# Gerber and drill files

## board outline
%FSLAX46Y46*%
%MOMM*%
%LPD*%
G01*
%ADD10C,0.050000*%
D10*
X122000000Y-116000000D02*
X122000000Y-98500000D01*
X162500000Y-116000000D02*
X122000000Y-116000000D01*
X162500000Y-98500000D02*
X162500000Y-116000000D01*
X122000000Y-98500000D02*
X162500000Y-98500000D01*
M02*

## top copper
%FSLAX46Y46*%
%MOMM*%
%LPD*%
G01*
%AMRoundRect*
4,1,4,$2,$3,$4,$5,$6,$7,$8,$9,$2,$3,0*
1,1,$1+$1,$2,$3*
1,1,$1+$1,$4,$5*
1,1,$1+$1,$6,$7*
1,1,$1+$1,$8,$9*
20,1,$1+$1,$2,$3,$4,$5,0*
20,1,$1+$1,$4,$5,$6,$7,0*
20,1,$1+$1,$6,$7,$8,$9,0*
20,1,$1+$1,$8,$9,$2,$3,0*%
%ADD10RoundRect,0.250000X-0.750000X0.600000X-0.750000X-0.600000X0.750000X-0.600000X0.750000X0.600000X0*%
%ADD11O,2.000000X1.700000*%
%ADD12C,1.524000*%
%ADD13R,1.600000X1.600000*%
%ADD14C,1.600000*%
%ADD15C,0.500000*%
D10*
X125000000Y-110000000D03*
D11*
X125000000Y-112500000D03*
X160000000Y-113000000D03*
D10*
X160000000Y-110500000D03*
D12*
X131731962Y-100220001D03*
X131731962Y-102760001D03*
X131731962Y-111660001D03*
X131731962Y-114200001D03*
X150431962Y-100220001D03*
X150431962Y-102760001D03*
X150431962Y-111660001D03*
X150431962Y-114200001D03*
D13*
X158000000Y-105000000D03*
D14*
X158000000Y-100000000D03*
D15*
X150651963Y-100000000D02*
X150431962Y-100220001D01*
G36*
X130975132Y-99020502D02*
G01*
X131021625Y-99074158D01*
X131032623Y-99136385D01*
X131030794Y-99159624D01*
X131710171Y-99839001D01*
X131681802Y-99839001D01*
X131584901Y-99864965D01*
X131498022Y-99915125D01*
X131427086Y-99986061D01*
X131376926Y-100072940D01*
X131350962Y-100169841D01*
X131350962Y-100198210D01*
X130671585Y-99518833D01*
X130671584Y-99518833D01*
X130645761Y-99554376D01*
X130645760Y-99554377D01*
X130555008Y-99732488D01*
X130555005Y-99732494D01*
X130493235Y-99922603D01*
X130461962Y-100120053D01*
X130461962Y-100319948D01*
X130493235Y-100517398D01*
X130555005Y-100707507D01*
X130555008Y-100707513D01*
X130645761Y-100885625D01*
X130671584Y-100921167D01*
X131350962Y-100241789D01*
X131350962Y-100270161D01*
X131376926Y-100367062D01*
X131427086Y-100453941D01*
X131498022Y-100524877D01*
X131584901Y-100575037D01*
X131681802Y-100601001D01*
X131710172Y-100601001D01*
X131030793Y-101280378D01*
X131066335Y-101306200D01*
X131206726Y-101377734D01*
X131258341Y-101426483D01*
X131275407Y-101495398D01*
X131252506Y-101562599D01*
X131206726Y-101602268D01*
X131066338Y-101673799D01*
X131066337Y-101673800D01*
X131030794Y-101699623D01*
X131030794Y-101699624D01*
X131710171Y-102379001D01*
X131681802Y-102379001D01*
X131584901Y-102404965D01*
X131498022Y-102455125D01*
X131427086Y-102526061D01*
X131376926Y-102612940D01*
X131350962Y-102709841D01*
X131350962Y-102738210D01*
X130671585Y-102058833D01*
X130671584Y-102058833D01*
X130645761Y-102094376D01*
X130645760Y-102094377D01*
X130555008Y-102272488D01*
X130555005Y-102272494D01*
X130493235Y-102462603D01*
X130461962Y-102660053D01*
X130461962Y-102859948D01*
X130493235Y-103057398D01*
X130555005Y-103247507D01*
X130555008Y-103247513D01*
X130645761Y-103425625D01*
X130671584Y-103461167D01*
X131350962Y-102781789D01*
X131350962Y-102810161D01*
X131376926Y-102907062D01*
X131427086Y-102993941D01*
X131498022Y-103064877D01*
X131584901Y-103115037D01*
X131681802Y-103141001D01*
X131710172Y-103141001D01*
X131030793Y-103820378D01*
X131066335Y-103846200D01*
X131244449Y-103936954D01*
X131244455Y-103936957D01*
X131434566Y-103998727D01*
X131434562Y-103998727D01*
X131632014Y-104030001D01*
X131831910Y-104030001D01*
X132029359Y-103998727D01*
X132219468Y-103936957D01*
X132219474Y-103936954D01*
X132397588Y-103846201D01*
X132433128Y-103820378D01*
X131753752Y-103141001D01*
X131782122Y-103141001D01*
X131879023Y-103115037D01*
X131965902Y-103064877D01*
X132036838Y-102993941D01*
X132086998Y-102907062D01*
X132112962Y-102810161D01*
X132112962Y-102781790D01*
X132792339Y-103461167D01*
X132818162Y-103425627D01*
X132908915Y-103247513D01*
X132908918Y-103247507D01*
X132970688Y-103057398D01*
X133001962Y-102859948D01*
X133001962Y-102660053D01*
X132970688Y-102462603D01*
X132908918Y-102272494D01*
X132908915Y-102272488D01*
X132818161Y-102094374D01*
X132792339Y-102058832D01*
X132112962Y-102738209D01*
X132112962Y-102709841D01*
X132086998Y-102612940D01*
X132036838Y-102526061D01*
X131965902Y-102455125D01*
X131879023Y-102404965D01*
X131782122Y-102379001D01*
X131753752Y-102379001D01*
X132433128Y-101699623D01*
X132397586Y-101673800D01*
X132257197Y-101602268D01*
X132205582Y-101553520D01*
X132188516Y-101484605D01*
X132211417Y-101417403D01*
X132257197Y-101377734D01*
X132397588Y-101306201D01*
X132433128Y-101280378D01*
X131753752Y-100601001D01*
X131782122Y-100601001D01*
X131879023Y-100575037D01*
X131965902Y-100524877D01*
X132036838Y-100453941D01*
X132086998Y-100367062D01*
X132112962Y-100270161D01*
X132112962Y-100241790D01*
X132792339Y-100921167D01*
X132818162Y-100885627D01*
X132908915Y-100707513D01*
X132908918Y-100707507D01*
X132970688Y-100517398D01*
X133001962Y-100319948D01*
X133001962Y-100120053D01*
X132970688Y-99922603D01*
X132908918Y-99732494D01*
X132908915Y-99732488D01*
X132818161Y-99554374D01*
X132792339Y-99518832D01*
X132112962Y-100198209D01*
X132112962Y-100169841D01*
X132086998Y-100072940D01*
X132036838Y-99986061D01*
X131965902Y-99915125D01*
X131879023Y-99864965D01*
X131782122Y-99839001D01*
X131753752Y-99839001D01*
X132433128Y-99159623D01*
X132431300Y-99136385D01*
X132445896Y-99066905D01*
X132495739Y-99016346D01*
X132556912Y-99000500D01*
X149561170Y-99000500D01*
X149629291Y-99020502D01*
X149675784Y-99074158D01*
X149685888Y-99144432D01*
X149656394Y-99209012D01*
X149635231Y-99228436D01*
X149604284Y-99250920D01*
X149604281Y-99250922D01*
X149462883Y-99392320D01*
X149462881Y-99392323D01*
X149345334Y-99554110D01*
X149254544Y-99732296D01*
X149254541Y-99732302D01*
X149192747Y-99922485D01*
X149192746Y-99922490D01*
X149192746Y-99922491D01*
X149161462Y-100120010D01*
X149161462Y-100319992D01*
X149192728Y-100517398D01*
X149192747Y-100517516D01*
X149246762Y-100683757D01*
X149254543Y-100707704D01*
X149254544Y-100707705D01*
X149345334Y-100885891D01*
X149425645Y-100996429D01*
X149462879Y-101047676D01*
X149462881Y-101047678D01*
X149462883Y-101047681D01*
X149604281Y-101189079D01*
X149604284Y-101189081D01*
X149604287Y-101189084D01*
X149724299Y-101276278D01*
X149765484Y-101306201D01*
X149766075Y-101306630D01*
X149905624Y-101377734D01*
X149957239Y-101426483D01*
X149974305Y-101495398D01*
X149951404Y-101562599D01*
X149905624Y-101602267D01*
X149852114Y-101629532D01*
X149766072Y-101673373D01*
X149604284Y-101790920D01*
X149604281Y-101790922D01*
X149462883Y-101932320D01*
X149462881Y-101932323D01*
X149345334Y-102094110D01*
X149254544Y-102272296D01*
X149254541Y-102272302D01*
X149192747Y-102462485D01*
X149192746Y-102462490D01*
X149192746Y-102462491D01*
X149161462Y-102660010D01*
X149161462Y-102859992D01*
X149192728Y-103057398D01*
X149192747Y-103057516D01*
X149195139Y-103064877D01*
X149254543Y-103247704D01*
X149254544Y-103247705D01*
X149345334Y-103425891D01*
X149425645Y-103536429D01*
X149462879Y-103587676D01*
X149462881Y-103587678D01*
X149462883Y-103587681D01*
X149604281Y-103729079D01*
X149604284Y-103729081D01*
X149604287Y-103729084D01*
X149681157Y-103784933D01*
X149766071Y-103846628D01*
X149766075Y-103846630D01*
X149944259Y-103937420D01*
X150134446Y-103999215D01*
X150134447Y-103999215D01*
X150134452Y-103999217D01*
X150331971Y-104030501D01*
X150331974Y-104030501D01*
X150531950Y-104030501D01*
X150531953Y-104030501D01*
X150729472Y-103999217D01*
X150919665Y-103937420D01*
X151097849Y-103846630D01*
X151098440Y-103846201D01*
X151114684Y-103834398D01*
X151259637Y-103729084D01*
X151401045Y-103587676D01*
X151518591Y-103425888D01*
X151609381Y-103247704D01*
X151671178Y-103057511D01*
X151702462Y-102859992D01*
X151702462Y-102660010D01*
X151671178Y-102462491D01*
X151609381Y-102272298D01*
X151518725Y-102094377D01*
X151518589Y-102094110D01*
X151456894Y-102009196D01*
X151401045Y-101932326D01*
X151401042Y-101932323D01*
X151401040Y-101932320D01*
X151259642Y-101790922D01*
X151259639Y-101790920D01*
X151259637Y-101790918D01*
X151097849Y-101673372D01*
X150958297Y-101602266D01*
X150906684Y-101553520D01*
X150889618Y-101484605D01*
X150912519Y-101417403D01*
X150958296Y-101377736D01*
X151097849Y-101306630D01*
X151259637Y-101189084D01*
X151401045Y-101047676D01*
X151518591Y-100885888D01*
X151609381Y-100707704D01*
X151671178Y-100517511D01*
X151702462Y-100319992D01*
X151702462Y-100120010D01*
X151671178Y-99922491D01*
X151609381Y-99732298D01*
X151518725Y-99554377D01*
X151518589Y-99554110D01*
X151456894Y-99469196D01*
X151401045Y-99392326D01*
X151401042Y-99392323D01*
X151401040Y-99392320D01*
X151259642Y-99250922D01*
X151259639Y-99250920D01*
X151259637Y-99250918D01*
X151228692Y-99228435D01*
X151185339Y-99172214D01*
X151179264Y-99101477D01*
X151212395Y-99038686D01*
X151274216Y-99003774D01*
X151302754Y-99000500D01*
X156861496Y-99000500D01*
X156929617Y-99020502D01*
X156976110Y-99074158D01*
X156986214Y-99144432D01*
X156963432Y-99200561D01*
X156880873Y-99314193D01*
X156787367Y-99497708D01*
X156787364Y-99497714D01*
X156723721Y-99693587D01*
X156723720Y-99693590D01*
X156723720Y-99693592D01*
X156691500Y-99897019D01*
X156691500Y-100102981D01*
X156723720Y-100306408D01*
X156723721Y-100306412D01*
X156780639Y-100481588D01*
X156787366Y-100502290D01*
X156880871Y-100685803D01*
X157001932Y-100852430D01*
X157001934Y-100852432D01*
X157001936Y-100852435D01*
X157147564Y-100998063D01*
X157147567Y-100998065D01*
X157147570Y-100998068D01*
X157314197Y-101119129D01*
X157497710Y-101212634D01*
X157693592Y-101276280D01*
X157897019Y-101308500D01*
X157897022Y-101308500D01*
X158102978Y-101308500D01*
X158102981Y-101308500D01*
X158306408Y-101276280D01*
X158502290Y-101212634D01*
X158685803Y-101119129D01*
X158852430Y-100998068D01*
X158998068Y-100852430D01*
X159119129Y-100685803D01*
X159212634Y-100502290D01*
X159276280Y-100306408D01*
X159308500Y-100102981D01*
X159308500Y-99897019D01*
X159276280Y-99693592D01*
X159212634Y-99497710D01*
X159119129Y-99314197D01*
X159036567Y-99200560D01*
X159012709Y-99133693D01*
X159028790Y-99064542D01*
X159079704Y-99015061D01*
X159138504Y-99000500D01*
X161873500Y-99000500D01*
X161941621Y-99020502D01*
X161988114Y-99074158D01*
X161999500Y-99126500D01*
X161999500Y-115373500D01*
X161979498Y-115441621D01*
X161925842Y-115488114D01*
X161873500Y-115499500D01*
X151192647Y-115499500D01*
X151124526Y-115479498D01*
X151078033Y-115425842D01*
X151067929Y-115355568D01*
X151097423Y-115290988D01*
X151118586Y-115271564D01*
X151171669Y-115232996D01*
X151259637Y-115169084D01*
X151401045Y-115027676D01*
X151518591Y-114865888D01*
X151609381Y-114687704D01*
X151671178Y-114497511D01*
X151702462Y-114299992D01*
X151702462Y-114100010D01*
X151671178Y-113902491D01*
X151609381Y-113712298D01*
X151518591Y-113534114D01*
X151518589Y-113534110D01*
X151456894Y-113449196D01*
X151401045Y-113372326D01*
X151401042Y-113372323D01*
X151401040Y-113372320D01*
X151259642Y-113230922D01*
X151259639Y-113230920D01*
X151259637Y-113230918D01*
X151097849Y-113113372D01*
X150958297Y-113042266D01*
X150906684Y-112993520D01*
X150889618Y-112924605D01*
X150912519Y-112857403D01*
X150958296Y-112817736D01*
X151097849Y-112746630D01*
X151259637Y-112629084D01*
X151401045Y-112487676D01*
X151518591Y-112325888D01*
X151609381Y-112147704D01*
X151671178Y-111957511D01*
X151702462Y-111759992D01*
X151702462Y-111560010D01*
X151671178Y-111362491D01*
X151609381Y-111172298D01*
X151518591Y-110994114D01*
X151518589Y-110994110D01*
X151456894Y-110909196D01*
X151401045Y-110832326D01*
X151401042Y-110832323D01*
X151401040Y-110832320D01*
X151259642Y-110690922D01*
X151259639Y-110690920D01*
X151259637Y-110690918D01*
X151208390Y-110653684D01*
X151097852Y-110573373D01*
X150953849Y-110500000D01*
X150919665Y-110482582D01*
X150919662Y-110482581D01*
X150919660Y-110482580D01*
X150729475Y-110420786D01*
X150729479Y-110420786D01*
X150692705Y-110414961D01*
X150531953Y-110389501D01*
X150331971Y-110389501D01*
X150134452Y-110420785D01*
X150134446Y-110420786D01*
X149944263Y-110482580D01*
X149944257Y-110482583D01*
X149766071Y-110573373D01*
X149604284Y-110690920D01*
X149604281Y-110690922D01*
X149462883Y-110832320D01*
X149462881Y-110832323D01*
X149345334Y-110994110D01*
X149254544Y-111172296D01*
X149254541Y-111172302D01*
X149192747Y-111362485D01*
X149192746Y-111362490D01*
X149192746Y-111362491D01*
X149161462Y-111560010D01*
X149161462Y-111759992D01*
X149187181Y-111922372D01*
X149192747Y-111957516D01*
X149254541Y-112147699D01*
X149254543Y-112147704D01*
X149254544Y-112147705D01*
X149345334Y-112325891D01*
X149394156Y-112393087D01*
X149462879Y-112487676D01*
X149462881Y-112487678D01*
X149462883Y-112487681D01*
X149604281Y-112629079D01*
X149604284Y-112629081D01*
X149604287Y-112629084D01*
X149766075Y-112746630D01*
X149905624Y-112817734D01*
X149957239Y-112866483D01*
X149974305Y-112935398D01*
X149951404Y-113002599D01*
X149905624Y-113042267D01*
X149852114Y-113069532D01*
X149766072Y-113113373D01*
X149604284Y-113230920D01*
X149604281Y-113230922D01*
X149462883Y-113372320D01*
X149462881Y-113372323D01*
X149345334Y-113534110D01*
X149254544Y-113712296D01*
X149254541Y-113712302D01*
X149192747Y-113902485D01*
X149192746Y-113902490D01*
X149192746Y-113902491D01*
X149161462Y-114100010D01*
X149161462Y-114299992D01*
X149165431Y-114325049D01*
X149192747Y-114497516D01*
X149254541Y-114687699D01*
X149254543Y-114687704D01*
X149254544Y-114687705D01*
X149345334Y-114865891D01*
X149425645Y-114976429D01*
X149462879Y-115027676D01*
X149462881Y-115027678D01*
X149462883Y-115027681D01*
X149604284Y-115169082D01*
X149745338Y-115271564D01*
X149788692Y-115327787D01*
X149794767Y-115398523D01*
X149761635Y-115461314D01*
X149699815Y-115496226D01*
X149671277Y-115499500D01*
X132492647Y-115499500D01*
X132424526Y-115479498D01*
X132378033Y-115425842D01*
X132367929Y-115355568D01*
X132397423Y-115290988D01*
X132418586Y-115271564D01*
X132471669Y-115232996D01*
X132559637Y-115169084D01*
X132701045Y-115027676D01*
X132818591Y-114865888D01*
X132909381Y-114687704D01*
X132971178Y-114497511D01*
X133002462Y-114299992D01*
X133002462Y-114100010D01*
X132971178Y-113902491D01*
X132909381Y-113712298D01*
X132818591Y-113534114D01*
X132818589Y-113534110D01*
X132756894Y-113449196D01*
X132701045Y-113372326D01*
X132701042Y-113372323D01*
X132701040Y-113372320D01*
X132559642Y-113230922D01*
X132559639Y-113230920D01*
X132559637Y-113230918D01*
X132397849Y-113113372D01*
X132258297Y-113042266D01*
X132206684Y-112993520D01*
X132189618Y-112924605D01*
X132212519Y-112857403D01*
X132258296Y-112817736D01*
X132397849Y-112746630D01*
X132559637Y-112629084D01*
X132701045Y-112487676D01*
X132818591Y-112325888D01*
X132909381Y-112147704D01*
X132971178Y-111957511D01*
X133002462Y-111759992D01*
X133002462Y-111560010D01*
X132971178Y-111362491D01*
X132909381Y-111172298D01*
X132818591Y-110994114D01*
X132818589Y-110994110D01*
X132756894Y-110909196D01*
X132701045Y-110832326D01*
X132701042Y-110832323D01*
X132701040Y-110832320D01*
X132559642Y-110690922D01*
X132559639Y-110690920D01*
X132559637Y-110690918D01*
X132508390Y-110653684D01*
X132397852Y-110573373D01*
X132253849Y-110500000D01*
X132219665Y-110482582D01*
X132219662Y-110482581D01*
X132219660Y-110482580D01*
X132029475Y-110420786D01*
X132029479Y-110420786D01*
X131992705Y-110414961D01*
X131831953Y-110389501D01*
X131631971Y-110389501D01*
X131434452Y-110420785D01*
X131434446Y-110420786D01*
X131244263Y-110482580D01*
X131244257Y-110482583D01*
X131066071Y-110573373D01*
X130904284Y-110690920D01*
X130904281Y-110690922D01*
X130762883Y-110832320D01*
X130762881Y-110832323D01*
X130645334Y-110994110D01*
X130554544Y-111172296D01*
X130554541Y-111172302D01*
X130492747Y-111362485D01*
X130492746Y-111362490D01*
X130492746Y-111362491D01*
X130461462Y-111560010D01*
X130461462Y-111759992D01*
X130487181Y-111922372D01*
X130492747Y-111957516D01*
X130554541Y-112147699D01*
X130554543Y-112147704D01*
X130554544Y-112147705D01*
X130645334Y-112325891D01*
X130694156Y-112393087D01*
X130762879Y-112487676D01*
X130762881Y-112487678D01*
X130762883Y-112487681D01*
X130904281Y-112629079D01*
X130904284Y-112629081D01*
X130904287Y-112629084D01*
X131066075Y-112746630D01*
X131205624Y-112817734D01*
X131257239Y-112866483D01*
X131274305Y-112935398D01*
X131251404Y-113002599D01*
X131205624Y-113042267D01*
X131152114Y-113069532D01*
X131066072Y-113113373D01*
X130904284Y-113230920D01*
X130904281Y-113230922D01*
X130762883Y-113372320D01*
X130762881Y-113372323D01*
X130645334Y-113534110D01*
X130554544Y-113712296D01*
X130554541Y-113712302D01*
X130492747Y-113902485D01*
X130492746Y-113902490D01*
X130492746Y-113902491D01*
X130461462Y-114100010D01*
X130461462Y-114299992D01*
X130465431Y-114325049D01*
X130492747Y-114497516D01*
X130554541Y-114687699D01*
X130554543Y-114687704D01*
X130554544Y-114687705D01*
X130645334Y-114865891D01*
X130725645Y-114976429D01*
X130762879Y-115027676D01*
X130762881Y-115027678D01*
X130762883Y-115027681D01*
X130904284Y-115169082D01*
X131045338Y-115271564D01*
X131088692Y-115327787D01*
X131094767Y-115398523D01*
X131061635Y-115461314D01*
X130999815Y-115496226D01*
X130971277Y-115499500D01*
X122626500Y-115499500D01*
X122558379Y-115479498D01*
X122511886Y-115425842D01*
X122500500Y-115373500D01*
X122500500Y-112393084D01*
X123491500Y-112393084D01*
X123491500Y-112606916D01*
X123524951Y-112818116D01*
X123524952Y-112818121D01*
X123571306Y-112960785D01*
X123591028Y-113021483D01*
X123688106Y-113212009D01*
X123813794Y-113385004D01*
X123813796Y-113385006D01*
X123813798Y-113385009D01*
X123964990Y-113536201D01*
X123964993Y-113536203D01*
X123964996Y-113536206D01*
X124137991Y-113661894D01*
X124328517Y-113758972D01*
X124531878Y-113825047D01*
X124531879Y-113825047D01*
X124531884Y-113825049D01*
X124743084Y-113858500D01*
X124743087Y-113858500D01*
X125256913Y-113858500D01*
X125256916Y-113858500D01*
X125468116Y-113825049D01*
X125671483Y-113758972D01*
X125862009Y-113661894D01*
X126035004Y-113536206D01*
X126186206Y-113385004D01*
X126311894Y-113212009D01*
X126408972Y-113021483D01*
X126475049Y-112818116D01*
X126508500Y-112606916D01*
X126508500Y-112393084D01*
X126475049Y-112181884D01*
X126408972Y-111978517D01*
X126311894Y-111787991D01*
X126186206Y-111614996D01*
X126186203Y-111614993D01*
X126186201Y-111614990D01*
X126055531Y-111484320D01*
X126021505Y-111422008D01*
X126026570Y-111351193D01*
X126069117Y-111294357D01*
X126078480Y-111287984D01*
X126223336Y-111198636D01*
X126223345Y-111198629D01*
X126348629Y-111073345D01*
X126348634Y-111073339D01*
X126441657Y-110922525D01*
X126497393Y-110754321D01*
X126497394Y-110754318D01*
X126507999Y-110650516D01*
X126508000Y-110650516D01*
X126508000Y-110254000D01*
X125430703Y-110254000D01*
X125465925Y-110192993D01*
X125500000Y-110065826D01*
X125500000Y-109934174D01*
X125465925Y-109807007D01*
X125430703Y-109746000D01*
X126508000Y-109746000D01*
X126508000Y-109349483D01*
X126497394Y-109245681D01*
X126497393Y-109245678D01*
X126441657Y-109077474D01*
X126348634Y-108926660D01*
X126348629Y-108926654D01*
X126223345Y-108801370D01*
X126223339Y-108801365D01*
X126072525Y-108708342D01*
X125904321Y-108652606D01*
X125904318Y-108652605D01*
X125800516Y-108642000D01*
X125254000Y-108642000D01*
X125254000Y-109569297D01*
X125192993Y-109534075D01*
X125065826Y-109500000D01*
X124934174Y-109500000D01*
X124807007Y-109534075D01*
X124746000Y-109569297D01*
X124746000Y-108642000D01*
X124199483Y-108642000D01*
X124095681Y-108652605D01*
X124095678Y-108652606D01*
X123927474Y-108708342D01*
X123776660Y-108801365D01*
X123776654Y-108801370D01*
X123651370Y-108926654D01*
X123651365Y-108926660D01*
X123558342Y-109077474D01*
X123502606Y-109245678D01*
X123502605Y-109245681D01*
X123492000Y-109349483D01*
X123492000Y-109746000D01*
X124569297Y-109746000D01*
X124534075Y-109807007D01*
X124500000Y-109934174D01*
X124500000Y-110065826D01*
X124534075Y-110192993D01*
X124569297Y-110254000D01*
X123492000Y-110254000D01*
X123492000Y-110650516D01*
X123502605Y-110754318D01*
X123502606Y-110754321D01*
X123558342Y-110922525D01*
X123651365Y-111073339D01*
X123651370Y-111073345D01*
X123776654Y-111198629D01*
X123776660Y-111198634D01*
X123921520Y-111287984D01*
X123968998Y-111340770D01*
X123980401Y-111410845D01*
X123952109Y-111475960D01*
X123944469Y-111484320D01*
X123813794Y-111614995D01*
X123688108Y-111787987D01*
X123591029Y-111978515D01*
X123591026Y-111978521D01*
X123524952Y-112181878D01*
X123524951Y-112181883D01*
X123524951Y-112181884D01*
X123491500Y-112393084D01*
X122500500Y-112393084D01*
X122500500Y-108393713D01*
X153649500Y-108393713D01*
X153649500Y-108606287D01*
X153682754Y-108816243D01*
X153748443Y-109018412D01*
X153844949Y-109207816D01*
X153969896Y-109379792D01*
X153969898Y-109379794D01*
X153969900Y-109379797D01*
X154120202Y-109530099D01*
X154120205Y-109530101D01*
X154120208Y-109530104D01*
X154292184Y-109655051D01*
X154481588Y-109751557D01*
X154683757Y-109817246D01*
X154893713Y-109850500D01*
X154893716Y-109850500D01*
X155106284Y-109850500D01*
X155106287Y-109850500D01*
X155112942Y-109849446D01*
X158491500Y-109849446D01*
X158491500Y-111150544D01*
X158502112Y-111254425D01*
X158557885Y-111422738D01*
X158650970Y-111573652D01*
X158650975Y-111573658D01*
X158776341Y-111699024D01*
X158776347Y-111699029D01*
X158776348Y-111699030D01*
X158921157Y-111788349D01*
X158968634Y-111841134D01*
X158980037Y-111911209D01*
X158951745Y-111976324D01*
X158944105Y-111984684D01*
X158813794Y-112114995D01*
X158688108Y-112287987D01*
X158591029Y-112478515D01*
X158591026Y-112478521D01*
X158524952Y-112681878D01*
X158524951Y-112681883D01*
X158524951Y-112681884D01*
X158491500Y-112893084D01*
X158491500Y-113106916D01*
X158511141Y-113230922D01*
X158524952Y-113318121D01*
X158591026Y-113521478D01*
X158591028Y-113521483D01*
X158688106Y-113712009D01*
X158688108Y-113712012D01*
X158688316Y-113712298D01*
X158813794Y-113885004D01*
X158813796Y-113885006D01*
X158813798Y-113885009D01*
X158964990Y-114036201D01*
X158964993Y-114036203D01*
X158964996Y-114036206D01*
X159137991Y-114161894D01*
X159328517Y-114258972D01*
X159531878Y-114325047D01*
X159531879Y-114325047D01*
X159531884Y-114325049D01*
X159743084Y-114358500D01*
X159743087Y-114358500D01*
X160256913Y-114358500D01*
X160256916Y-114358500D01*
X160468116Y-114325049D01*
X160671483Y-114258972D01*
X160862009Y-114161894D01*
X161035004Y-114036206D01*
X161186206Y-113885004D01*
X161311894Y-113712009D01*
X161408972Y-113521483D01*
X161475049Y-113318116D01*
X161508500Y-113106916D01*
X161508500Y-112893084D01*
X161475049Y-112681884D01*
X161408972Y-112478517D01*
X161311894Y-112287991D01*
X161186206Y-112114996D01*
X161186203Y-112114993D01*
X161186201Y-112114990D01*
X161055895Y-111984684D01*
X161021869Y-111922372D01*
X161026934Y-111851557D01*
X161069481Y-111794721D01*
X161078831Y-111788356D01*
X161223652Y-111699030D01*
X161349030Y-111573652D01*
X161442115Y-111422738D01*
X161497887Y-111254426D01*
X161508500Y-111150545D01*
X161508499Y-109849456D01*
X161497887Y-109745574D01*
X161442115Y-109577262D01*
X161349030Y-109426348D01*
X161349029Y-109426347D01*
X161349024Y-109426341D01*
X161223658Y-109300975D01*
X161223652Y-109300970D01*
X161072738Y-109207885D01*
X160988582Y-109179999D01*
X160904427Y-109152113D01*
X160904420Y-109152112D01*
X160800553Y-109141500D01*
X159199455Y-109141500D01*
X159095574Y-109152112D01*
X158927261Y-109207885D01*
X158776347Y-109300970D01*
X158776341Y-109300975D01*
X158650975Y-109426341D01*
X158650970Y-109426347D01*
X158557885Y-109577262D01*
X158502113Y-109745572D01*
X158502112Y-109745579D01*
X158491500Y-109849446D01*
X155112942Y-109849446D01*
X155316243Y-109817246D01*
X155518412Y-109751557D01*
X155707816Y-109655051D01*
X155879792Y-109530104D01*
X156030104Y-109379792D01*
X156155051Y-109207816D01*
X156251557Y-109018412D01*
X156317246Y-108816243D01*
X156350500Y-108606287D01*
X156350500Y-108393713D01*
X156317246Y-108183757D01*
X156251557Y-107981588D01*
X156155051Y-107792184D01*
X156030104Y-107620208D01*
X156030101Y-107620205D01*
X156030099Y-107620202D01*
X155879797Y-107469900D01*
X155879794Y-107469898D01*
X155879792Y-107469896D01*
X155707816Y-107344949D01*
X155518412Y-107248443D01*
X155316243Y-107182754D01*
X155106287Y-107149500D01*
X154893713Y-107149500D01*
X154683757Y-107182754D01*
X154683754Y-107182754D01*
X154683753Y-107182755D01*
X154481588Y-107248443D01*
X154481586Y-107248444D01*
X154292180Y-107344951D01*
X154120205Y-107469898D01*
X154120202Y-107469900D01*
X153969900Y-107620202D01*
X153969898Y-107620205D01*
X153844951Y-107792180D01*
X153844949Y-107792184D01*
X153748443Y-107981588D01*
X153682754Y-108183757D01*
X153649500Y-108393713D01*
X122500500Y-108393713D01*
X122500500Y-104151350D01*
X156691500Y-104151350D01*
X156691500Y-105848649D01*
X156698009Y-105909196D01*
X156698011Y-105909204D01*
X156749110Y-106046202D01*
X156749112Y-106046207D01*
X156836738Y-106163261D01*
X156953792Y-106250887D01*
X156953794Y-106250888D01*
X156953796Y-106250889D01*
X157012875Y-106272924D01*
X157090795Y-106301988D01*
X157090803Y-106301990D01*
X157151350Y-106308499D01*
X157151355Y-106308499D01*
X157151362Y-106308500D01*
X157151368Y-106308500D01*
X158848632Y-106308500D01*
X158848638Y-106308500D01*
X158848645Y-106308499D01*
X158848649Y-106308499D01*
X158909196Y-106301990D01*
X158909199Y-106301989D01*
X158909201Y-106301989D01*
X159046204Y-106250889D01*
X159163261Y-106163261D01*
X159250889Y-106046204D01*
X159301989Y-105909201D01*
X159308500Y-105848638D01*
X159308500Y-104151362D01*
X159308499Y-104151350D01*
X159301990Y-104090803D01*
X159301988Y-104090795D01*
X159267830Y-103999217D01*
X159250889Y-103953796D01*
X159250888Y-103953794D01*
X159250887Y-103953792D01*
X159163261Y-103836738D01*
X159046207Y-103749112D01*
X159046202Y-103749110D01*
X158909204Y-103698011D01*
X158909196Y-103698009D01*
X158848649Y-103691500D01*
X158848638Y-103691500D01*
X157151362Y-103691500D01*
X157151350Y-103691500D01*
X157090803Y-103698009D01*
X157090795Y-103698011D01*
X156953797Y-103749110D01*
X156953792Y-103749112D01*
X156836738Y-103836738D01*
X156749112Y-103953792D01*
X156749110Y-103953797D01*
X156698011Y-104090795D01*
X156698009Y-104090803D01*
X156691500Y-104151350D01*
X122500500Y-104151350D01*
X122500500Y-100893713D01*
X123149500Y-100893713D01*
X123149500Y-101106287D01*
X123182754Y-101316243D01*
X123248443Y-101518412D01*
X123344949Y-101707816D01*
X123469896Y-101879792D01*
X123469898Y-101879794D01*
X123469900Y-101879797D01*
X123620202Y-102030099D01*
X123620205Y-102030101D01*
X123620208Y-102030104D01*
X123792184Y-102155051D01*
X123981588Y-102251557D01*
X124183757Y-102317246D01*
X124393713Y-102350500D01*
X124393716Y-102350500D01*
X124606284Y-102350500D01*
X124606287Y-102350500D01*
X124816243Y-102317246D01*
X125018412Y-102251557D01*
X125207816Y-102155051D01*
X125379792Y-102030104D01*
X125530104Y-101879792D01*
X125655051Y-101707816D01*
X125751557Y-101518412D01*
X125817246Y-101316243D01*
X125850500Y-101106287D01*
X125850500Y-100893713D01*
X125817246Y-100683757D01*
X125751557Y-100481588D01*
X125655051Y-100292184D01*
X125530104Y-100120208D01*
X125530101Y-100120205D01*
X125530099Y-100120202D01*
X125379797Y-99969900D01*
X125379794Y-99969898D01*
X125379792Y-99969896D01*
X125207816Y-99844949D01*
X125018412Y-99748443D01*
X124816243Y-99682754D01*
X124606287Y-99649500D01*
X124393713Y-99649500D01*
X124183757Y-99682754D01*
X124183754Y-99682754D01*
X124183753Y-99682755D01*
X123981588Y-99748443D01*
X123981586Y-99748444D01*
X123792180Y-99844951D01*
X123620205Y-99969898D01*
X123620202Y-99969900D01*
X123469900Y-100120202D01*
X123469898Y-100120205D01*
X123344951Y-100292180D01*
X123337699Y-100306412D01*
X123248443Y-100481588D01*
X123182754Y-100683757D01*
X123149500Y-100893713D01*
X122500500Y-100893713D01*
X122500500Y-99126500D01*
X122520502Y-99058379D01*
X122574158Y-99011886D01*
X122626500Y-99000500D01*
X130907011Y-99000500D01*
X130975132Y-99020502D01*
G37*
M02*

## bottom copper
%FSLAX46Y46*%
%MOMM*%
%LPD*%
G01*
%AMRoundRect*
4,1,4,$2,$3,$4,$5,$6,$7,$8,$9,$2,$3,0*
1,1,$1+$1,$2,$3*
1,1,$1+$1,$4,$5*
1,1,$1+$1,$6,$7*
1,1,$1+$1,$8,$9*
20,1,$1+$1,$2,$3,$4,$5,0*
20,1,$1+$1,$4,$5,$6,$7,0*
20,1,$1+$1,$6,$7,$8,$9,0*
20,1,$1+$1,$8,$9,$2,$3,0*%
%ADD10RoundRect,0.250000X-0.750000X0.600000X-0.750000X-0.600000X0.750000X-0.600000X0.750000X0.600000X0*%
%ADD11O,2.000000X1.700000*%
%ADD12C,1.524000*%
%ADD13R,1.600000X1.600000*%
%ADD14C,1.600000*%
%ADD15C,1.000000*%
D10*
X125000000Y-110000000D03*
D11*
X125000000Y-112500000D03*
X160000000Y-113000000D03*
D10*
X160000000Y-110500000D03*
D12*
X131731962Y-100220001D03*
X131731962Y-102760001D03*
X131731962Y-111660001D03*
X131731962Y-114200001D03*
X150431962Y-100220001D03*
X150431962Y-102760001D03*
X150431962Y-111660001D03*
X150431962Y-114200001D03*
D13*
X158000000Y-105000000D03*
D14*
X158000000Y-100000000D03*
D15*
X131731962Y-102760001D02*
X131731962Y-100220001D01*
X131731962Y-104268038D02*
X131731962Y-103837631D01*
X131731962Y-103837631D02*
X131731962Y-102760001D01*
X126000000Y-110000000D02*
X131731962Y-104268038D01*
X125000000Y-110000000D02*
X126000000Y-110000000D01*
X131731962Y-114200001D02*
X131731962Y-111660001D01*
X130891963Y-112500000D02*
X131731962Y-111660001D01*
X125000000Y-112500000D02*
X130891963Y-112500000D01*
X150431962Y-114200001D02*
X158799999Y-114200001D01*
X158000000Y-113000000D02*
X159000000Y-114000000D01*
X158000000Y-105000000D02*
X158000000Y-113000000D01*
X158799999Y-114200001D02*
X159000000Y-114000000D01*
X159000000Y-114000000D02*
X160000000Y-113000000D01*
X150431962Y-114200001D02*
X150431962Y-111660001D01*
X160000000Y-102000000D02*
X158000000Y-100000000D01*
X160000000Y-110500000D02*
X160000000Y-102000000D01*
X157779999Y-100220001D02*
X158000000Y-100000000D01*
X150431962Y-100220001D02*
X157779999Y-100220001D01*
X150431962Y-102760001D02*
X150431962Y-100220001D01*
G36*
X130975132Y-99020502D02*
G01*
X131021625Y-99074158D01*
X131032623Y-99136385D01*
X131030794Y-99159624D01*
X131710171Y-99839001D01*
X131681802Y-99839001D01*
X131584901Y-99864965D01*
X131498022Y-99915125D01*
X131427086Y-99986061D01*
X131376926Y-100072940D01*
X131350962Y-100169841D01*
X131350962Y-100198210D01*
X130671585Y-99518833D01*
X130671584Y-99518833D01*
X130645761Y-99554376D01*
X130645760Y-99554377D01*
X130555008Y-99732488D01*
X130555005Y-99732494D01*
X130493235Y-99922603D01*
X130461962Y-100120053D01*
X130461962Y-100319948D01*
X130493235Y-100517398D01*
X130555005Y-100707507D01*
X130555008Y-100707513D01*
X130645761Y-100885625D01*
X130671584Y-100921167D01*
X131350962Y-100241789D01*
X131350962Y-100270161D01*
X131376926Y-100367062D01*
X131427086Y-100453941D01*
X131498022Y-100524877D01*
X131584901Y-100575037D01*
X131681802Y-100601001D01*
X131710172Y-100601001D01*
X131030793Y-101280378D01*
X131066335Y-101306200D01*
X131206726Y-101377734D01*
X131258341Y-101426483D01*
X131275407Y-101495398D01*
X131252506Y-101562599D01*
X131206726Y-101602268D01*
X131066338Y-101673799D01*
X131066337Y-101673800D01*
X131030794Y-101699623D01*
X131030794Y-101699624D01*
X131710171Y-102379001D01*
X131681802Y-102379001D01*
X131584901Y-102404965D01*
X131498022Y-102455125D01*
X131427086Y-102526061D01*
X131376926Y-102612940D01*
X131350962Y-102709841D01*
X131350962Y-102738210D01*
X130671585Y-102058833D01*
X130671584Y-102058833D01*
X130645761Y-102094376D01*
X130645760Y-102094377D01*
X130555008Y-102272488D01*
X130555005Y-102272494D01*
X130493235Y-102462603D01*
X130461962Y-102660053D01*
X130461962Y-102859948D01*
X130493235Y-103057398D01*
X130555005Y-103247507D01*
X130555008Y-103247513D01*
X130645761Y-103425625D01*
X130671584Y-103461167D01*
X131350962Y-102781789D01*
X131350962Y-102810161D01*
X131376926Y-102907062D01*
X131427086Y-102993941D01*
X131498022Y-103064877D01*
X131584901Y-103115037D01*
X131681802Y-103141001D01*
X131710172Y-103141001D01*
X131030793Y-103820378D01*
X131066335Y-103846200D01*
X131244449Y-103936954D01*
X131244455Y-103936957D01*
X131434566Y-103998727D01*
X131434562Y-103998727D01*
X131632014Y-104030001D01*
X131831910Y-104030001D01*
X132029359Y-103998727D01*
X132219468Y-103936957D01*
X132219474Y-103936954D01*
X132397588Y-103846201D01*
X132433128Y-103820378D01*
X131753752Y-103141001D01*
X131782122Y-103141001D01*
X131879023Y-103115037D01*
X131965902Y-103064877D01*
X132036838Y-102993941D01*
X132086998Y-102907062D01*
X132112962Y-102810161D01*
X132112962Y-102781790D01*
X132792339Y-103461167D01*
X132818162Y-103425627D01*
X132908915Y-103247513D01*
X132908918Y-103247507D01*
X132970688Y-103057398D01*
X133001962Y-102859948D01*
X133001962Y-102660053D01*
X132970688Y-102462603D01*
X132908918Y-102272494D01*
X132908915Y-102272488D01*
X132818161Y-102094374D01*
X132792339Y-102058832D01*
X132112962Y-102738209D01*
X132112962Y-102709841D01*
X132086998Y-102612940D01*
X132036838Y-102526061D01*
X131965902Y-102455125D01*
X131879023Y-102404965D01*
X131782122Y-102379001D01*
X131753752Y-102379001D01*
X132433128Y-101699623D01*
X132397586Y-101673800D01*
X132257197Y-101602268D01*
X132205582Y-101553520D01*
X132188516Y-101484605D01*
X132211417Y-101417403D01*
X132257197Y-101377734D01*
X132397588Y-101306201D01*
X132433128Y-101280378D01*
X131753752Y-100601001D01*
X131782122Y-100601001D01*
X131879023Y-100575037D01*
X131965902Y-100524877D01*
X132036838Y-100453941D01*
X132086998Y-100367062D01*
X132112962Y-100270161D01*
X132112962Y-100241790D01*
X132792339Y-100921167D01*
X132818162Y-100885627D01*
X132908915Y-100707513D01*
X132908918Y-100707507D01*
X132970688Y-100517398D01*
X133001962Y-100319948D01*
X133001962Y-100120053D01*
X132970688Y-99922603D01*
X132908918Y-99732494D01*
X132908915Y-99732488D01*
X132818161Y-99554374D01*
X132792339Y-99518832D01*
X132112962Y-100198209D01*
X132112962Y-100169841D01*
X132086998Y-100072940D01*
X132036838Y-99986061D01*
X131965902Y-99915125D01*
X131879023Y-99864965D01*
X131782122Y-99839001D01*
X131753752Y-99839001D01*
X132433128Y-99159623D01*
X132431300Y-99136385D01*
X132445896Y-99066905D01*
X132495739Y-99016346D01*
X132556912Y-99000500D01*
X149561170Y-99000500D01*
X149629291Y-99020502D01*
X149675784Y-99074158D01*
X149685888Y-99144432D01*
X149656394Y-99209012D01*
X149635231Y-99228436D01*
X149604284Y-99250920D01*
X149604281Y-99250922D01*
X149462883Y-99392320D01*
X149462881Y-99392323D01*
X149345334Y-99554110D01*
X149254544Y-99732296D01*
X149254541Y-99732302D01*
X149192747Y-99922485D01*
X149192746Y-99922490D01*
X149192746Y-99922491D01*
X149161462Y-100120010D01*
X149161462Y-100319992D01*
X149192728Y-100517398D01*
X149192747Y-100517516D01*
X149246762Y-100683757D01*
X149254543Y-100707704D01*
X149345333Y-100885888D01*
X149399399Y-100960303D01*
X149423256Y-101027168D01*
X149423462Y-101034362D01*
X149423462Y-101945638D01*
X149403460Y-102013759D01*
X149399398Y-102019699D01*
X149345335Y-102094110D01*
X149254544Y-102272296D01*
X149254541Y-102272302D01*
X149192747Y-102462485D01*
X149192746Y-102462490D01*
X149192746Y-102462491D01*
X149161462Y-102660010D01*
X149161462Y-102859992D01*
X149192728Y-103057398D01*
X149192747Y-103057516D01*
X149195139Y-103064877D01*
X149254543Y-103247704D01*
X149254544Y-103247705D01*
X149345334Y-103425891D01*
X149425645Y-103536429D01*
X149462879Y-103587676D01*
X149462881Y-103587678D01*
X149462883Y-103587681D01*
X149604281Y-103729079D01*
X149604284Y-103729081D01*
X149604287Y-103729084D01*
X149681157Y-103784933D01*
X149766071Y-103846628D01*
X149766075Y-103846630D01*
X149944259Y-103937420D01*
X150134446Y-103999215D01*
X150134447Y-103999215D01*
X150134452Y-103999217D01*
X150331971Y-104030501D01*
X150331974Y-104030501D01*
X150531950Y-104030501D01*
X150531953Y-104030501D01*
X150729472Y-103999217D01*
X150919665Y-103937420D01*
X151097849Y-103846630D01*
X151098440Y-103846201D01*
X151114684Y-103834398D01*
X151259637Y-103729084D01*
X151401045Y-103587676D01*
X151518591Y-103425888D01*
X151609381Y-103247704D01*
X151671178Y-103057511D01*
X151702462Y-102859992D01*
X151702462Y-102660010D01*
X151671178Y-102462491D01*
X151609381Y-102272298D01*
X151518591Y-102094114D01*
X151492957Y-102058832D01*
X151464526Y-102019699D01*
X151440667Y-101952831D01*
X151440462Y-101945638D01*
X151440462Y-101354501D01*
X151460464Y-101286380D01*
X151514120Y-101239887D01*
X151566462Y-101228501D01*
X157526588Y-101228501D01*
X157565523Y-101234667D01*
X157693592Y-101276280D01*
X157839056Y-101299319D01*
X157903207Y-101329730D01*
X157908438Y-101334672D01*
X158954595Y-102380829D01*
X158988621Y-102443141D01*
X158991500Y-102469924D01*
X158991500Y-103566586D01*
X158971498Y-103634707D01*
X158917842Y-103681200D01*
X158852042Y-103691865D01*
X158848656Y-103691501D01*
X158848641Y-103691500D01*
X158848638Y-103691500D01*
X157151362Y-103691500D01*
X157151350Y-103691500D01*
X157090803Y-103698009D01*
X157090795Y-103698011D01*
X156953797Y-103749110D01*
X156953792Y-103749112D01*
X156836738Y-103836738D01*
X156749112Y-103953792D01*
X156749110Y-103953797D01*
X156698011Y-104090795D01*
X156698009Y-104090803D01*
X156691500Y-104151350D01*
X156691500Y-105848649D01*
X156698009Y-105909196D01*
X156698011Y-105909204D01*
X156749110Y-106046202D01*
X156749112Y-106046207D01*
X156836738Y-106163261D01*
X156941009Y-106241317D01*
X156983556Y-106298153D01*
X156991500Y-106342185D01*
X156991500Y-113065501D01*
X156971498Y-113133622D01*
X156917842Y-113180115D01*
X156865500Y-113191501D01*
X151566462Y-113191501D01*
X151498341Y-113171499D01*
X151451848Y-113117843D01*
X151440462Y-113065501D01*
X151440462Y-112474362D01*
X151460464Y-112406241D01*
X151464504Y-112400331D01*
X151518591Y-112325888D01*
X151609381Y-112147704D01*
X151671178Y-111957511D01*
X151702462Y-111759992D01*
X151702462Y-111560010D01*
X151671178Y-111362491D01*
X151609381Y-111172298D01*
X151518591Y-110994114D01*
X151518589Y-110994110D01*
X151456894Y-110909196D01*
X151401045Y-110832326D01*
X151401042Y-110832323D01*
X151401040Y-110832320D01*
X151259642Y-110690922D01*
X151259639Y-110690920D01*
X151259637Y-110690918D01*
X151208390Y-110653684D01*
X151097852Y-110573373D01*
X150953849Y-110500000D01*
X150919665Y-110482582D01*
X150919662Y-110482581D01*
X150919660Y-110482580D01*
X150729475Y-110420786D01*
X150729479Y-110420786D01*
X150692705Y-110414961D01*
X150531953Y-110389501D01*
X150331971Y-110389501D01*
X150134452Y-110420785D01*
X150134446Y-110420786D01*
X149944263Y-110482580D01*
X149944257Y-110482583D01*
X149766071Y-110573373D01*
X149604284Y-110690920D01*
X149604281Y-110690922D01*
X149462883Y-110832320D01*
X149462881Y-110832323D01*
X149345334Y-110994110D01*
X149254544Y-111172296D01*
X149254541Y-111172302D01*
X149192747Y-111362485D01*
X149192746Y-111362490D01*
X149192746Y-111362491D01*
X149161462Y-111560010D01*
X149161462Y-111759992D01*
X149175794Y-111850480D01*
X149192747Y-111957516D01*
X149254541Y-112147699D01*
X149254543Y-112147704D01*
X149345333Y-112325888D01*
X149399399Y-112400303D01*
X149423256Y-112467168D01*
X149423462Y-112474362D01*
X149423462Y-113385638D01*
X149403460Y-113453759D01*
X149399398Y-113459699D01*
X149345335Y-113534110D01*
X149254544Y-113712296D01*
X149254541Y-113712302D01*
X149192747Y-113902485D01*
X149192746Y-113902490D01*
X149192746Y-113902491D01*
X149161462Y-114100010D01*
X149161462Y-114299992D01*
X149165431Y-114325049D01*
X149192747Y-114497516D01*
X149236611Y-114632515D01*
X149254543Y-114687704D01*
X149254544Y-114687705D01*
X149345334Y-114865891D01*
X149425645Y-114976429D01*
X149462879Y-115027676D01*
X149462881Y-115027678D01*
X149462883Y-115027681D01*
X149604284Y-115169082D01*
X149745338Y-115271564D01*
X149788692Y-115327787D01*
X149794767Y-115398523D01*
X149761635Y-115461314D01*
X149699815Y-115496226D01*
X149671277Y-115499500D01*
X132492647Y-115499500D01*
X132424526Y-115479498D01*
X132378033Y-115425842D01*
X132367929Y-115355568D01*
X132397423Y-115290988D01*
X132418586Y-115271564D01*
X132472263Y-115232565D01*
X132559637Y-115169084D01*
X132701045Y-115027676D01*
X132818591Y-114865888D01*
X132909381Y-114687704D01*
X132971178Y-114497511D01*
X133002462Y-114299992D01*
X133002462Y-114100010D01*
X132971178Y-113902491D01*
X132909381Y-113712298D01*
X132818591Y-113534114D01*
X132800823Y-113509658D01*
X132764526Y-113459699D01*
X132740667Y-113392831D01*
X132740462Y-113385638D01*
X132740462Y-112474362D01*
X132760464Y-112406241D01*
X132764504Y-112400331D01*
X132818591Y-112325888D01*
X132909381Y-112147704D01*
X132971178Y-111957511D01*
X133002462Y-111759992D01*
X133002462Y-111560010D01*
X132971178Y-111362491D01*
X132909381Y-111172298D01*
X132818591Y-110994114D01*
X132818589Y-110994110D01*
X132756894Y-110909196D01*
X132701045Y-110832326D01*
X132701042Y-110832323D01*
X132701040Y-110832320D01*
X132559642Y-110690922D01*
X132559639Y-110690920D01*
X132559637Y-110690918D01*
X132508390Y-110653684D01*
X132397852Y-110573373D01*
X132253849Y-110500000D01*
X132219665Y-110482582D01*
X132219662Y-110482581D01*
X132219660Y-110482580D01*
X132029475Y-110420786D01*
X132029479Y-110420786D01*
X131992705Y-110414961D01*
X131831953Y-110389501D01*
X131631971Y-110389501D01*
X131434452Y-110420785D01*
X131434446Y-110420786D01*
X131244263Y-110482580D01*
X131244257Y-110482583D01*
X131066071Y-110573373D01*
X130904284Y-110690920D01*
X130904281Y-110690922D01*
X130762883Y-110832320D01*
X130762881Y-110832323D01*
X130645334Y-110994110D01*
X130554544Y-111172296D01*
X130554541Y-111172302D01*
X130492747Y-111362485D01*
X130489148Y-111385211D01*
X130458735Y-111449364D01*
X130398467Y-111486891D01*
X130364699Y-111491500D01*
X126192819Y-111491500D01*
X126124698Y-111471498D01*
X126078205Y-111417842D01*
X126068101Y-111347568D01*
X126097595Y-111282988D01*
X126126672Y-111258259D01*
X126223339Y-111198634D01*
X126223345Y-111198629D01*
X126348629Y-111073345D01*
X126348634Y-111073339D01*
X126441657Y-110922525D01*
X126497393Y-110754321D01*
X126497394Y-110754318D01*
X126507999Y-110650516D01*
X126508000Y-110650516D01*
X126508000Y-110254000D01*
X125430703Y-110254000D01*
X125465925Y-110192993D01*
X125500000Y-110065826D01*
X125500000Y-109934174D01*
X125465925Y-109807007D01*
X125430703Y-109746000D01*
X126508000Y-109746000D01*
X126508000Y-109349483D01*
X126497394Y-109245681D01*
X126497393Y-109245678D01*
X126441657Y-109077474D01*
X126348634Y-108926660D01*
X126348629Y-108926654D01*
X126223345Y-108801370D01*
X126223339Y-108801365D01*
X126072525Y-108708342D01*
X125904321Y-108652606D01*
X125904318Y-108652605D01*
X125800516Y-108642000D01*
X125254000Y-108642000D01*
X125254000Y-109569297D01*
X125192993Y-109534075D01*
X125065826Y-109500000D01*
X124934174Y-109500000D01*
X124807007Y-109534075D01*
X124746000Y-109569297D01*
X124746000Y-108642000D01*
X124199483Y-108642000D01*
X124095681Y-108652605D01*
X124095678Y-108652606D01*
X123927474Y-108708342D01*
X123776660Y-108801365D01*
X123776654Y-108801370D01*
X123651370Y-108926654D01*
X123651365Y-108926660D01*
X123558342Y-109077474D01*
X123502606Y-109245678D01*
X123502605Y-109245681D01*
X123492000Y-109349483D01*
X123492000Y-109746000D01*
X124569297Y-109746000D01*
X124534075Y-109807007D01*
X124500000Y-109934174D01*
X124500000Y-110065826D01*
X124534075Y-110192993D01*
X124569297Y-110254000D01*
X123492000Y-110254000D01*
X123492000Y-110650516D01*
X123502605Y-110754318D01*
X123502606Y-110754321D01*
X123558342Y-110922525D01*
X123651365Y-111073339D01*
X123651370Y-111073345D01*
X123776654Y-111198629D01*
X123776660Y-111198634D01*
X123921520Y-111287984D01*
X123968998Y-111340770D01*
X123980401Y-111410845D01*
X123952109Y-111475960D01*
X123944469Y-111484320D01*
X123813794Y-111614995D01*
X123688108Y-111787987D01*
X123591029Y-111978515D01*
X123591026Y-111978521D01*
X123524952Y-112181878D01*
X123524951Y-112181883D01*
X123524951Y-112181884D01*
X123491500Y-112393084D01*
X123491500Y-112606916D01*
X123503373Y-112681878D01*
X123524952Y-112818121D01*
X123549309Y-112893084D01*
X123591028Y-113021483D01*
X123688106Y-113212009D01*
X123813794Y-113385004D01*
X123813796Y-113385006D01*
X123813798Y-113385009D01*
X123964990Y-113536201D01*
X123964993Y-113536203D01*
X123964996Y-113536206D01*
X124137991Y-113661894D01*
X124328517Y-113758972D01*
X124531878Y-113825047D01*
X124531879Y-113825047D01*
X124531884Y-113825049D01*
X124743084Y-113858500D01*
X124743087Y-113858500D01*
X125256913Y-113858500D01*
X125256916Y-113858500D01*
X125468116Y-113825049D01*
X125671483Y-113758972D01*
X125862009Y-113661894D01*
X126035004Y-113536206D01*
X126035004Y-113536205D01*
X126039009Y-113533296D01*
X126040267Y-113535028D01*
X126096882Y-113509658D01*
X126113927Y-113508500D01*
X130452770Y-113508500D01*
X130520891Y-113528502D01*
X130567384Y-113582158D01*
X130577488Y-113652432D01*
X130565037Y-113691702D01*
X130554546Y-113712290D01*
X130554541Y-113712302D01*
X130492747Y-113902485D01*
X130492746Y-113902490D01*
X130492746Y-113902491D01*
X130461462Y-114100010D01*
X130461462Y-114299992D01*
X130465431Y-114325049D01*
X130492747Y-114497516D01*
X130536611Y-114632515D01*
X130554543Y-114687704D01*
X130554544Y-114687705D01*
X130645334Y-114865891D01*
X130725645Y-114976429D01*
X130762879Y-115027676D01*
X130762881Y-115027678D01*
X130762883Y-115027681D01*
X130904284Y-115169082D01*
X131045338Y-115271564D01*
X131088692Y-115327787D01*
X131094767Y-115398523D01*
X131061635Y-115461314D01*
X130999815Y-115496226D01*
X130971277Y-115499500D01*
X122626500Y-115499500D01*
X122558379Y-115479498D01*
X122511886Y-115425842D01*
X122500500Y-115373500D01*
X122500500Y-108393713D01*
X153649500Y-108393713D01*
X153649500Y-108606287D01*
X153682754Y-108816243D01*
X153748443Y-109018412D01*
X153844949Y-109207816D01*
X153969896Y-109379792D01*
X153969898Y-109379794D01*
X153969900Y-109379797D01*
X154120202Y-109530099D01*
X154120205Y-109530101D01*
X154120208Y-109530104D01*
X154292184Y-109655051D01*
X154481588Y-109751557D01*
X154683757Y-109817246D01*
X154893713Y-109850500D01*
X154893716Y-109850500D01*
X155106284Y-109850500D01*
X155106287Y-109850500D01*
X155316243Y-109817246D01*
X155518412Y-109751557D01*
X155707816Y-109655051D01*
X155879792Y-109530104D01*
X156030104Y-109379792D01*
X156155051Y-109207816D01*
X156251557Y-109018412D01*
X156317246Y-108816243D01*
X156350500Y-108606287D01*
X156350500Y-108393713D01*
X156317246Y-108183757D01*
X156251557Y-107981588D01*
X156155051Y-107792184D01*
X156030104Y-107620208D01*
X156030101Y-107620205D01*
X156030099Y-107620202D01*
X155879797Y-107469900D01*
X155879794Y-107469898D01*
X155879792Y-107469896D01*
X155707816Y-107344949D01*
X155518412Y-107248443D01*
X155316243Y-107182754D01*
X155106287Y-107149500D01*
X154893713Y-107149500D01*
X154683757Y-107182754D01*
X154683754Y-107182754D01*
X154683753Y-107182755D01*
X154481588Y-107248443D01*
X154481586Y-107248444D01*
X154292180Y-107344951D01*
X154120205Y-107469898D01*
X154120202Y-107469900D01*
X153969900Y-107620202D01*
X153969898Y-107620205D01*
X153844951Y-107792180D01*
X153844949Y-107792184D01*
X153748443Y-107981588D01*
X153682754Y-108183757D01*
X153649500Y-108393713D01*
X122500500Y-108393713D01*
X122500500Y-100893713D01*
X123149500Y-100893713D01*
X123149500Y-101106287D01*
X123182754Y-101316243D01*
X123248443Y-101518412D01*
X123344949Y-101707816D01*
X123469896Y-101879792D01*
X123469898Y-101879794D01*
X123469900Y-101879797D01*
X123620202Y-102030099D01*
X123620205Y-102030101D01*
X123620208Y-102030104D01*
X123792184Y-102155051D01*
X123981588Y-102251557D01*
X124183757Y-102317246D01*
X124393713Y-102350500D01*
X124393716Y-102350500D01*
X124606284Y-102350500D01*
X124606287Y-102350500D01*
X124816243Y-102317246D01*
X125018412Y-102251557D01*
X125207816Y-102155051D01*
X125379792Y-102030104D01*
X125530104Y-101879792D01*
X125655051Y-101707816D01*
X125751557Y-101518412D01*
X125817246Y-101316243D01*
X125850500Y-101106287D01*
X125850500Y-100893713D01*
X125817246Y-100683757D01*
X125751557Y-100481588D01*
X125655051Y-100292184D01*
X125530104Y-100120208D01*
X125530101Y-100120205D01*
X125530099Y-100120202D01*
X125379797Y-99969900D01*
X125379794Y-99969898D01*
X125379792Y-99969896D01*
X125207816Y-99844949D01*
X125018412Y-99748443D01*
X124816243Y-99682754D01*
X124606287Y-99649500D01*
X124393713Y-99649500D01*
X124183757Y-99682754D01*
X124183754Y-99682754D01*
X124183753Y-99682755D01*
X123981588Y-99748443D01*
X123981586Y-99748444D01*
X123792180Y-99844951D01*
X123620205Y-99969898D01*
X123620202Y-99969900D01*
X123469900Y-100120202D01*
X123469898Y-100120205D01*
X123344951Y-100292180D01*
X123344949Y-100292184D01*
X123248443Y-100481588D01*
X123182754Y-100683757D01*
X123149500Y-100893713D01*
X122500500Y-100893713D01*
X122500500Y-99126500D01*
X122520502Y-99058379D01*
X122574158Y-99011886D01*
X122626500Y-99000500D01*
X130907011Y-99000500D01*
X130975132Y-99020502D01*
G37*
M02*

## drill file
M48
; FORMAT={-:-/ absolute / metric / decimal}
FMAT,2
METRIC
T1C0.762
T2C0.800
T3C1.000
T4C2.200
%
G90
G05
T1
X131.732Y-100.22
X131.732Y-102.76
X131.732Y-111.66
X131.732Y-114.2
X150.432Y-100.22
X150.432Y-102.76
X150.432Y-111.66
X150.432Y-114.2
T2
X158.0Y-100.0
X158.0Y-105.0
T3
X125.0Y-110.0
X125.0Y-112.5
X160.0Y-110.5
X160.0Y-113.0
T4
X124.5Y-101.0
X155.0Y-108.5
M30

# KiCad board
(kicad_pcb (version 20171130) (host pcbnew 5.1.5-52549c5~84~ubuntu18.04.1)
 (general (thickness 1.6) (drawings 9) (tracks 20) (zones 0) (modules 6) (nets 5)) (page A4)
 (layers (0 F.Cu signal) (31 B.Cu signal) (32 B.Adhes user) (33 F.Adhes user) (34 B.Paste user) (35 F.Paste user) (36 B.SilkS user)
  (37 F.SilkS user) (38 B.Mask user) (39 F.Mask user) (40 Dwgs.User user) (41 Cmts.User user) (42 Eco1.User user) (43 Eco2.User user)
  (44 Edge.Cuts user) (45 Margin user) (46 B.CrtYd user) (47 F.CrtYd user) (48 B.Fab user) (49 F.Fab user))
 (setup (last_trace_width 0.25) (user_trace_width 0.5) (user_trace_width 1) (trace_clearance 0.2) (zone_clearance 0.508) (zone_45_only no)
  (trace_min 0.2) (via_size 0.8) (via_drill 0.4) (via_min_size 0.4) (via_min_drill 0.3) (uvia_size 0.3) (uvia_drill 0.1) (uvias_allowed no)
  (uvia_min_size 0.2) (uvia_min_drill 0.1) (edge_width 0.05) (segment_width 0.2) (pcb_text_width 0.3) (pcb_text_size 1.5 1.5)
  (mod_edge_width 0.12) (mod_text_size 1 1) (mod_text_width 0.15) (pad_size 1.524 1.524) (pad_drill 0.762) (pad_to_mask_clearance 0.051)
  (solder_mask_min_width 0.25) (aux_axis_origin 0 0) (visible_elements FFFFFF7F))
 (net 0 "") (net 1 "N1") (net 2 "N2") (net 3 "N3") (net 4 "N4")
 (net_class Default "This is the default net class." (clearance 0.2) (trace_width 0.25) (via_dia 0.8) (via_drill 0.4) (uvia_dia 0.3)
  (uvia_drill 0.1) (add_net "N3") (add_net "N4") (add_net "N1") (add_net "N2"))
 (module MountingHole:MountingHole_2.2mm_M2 (layer F.Cu) (at 155 108.5)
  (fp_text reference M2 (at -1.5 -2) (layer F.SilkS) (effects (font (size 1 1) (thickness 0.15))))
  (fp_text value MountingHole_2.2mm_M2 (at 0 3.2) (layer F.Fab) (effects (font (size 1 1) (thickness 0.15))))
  (pad 1 np_thru_hole circle (at 0 0) (size 2.2 2.2) (drill 2.2) (layers *.Cu *.Mask)))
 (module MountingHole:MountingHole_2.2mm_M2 (layer F.Cu) (at 124.5 101)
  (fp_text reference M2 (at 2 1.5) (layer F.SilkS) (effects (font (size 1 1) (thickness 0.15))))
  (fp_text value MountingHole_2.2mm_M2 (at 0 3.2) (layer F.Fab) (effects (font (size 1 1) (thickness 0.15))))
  (pad 1 np_thru_hole circle (at 0 0) (size 2.2 2.2) (drill 2.2) (layers *.Cu *.Mask)))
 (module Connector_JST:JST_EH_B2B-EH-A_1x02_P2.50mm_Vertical (layer F.Cu) (at 125 110 270)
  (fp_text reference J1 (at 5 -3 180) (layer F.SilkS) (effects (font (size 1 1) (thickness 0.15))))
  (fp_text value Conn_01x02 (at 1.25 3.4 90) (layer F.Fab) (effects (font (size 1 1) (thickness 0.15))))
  (pad 1 thru_hole roundrect (at 0 0 270) (size 1.7 2) (drill 1) (layers *.Cu *.Mask) (roundrect_rratio 0.147059) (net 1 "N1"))
  (pad 2 thru_hole oval (at 2.5 0 270) (size 1.7 2) (drill 1) (layers *.Cu *.Mask) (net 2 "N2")))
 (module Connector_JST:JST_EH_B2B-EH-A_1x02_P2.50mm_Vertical (layer F.Cu) (at 160 110.5 270)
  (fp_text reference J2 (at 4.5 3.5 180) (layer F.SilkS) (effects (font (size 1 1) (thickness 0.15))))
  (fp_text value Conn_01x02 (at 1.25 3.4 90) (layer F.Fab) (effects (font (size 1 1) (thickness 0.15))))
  (pad 2 thru_hole oval (at 2.5 0 270) (size 1.7 2) (drill 1) (layers *.Cu *.Mask) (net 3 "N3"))
  (pad 1 thru_hole roundrect (at 0 0 270) (size 1.7 2) (drill 1) (layers *.Cu *.Mask) (roundrect_rratio 0.147059) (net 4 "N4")))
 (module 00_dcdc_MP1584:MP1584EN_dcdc (layer F.Cu) (at 141.081962 107.210001)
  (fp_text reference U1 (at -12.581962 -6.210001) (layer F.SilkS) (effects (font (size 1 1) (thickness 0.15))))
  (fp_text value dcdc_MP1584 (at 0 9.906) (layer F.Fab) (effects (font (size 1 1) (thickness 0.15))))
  (pad 1 thru_hole circle (at -9.35 -6.99) (size 1.524 1.524) (drill 0.762) (layers *.Cu *.Mask) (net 1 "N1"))
  (pad 2 thru_hole circle (at -9.35 -4.45) (size 1.524 1.524) (drill 0.762) (layers *.Cu *.Mask) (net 1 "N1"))
  (pad 3 thru_hole circle (at -9.35 4.45) (size 1.524 1.524) (drill 0.762) (layers *.Cu *.Mask) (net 2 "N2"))
  (pad 4 thru_hole circle (at -9.35 6.99) (size 1.524 1.524) (drill 0.762) (layers *.Cu *.Mask) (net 2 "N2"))
  (pad 5 thru_hole circle (at 9.35 -6.99) (size 1.524 1.524) (drill 0.762) (layers *.Cu *.Mask) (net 4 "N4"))
  (pad 6 thru_hole circle (at 9.35 -4.45) (size 1.524 1.524) (drill 0.762) (layers *.Cu *.Mask) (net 4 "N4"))
  (pad 7 thru_hole circle (at 9.35 4.45) (size 1.524 1.524) (drill 0.762) (layers *.Cu *.Mask) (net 3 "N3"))
  (pad 8 thru_hole circle (at 9.35 6.99) (size 1.524 1.524) (drill 0.762) (layers *.Cu *.Mask) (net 3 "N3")))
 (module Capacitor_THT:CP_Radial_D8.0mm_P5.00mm (layer F.Cu) (at 158 105 90)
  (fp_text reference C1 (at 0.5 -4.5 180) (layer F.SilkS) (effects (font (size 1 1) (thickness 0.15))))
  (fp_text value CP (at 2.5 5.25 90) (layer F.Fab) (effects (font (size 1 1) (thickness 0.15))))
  (pad 1 thru_hole rect (at 0 0 90) (size 1.6 1.6) (drill 0.8) (layers *.Cu *.Mask) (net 3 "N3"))
  (pad 2 thru_hole circle (at 5 0 90) (size 1.6 1.6) (drill 0.8) (layers *.Cu *.Mask) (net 4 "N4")))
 (gr_line (start 122 116) (end 122 98.5) (layer Edge.Cuts) (width 0.05))
 (gr_line (start 162.5 116) (end 122 116) (layer Edge.Cuts) (width 0.05))
 (gr_line (start 162.5 98.5) (end 162.5 116) (layer Edge.Cuts) (width 0.05))
 (gr_line (start 122 98.5) (end 162.5 98.5) (layer Edge.Cuts) (width 0.05))
 (segment (start 131.731962 102.760001) (end 131.731962 100.220001) (width 1) (layer B.Cu) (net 1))
 (segment (start 131.731962 104.268038) (end 131.731962 103.837631) (width 1) (layer B.Cu) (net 1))
 (segment (start 131.731962 103.837631) (end 131.731962 102.760001) (width 1) (layer B.Cu) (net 1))
 (segment (start 126 110) (end 131.731962 104.268038) (width 1) (layer B.Cu) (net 1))
 (segment (start 125 110) (end 126 110) (width 1) (layer B.Cu) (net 1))
 (segment (start 131.731962 114.200001) (end 131.731962 111.660001) (width 1) (layer B.Cu) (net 2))
 (segment (start 130.891963 112.5) (end 131.731962 111.660001) (width 1) (layer B.Cu) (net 2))
 (segment (start 125 112.5) (end 130.891963 112.5) (width 1) (layer B.Cu) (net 2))
 (segment (start 150.431962 114.200001) (end 158.799999 114.200001) (width 1) (layer B.Cu) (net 3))
 (segment (start 158 113) (end 159 114) (width 1) (layer B.Cu) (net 3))
 (segment (start 158 105) (end 158 113) (width 1) (layer B.Cu) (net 3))
 (segment (start 158.799999 114.200001) (end 159 114) (width 1) (layer B.Cu) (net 3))
 (segment (start 159 114) (end 160 113) (width 1) (layer B.Cu) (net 3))
 (segment (start 150.431962 114.200001) (end 150.431962 111.660001) (width 1) (layer B.Cu) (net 3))
 (segment (start 150.651963 100) (end 150.431962 100.220001) (width 0.5) (layer F.Cu) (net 4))
 (segment (start 160 102) (end 158 100) (width 1) (layer B.Cu) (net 4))
 (segment (start 160 110.5) (end 160 102) (width 1) (layer B.Cu) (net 4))
 (segment (start 157.779999 100.220001) (end 158 100) (width 1) (layer B.Cu) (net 4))
 (segment (start 150.431962 100.220001) (end 157.779999 100.220001) (width 1) (layer B.Cu) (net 4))
 (segment (start 150.431962 102.760001) (end 150.431962 100.220001) (width 1) (layer B.Cu) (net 4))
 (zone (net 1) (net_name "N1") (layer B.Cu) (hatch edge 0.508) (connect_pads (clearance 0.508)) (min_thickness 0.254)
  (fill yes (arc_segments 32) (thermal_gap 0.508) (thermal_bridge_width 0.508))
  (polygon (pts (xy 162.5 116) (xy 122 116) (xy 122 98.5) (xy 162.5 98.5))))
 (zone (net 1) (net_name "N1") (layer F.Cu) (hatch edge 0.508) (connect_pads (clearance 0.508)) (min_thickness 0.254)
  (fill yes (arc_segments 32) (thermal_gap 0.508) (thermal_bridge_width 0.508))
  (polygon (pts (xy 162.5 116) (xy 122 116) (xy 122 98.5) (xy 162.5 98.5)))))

